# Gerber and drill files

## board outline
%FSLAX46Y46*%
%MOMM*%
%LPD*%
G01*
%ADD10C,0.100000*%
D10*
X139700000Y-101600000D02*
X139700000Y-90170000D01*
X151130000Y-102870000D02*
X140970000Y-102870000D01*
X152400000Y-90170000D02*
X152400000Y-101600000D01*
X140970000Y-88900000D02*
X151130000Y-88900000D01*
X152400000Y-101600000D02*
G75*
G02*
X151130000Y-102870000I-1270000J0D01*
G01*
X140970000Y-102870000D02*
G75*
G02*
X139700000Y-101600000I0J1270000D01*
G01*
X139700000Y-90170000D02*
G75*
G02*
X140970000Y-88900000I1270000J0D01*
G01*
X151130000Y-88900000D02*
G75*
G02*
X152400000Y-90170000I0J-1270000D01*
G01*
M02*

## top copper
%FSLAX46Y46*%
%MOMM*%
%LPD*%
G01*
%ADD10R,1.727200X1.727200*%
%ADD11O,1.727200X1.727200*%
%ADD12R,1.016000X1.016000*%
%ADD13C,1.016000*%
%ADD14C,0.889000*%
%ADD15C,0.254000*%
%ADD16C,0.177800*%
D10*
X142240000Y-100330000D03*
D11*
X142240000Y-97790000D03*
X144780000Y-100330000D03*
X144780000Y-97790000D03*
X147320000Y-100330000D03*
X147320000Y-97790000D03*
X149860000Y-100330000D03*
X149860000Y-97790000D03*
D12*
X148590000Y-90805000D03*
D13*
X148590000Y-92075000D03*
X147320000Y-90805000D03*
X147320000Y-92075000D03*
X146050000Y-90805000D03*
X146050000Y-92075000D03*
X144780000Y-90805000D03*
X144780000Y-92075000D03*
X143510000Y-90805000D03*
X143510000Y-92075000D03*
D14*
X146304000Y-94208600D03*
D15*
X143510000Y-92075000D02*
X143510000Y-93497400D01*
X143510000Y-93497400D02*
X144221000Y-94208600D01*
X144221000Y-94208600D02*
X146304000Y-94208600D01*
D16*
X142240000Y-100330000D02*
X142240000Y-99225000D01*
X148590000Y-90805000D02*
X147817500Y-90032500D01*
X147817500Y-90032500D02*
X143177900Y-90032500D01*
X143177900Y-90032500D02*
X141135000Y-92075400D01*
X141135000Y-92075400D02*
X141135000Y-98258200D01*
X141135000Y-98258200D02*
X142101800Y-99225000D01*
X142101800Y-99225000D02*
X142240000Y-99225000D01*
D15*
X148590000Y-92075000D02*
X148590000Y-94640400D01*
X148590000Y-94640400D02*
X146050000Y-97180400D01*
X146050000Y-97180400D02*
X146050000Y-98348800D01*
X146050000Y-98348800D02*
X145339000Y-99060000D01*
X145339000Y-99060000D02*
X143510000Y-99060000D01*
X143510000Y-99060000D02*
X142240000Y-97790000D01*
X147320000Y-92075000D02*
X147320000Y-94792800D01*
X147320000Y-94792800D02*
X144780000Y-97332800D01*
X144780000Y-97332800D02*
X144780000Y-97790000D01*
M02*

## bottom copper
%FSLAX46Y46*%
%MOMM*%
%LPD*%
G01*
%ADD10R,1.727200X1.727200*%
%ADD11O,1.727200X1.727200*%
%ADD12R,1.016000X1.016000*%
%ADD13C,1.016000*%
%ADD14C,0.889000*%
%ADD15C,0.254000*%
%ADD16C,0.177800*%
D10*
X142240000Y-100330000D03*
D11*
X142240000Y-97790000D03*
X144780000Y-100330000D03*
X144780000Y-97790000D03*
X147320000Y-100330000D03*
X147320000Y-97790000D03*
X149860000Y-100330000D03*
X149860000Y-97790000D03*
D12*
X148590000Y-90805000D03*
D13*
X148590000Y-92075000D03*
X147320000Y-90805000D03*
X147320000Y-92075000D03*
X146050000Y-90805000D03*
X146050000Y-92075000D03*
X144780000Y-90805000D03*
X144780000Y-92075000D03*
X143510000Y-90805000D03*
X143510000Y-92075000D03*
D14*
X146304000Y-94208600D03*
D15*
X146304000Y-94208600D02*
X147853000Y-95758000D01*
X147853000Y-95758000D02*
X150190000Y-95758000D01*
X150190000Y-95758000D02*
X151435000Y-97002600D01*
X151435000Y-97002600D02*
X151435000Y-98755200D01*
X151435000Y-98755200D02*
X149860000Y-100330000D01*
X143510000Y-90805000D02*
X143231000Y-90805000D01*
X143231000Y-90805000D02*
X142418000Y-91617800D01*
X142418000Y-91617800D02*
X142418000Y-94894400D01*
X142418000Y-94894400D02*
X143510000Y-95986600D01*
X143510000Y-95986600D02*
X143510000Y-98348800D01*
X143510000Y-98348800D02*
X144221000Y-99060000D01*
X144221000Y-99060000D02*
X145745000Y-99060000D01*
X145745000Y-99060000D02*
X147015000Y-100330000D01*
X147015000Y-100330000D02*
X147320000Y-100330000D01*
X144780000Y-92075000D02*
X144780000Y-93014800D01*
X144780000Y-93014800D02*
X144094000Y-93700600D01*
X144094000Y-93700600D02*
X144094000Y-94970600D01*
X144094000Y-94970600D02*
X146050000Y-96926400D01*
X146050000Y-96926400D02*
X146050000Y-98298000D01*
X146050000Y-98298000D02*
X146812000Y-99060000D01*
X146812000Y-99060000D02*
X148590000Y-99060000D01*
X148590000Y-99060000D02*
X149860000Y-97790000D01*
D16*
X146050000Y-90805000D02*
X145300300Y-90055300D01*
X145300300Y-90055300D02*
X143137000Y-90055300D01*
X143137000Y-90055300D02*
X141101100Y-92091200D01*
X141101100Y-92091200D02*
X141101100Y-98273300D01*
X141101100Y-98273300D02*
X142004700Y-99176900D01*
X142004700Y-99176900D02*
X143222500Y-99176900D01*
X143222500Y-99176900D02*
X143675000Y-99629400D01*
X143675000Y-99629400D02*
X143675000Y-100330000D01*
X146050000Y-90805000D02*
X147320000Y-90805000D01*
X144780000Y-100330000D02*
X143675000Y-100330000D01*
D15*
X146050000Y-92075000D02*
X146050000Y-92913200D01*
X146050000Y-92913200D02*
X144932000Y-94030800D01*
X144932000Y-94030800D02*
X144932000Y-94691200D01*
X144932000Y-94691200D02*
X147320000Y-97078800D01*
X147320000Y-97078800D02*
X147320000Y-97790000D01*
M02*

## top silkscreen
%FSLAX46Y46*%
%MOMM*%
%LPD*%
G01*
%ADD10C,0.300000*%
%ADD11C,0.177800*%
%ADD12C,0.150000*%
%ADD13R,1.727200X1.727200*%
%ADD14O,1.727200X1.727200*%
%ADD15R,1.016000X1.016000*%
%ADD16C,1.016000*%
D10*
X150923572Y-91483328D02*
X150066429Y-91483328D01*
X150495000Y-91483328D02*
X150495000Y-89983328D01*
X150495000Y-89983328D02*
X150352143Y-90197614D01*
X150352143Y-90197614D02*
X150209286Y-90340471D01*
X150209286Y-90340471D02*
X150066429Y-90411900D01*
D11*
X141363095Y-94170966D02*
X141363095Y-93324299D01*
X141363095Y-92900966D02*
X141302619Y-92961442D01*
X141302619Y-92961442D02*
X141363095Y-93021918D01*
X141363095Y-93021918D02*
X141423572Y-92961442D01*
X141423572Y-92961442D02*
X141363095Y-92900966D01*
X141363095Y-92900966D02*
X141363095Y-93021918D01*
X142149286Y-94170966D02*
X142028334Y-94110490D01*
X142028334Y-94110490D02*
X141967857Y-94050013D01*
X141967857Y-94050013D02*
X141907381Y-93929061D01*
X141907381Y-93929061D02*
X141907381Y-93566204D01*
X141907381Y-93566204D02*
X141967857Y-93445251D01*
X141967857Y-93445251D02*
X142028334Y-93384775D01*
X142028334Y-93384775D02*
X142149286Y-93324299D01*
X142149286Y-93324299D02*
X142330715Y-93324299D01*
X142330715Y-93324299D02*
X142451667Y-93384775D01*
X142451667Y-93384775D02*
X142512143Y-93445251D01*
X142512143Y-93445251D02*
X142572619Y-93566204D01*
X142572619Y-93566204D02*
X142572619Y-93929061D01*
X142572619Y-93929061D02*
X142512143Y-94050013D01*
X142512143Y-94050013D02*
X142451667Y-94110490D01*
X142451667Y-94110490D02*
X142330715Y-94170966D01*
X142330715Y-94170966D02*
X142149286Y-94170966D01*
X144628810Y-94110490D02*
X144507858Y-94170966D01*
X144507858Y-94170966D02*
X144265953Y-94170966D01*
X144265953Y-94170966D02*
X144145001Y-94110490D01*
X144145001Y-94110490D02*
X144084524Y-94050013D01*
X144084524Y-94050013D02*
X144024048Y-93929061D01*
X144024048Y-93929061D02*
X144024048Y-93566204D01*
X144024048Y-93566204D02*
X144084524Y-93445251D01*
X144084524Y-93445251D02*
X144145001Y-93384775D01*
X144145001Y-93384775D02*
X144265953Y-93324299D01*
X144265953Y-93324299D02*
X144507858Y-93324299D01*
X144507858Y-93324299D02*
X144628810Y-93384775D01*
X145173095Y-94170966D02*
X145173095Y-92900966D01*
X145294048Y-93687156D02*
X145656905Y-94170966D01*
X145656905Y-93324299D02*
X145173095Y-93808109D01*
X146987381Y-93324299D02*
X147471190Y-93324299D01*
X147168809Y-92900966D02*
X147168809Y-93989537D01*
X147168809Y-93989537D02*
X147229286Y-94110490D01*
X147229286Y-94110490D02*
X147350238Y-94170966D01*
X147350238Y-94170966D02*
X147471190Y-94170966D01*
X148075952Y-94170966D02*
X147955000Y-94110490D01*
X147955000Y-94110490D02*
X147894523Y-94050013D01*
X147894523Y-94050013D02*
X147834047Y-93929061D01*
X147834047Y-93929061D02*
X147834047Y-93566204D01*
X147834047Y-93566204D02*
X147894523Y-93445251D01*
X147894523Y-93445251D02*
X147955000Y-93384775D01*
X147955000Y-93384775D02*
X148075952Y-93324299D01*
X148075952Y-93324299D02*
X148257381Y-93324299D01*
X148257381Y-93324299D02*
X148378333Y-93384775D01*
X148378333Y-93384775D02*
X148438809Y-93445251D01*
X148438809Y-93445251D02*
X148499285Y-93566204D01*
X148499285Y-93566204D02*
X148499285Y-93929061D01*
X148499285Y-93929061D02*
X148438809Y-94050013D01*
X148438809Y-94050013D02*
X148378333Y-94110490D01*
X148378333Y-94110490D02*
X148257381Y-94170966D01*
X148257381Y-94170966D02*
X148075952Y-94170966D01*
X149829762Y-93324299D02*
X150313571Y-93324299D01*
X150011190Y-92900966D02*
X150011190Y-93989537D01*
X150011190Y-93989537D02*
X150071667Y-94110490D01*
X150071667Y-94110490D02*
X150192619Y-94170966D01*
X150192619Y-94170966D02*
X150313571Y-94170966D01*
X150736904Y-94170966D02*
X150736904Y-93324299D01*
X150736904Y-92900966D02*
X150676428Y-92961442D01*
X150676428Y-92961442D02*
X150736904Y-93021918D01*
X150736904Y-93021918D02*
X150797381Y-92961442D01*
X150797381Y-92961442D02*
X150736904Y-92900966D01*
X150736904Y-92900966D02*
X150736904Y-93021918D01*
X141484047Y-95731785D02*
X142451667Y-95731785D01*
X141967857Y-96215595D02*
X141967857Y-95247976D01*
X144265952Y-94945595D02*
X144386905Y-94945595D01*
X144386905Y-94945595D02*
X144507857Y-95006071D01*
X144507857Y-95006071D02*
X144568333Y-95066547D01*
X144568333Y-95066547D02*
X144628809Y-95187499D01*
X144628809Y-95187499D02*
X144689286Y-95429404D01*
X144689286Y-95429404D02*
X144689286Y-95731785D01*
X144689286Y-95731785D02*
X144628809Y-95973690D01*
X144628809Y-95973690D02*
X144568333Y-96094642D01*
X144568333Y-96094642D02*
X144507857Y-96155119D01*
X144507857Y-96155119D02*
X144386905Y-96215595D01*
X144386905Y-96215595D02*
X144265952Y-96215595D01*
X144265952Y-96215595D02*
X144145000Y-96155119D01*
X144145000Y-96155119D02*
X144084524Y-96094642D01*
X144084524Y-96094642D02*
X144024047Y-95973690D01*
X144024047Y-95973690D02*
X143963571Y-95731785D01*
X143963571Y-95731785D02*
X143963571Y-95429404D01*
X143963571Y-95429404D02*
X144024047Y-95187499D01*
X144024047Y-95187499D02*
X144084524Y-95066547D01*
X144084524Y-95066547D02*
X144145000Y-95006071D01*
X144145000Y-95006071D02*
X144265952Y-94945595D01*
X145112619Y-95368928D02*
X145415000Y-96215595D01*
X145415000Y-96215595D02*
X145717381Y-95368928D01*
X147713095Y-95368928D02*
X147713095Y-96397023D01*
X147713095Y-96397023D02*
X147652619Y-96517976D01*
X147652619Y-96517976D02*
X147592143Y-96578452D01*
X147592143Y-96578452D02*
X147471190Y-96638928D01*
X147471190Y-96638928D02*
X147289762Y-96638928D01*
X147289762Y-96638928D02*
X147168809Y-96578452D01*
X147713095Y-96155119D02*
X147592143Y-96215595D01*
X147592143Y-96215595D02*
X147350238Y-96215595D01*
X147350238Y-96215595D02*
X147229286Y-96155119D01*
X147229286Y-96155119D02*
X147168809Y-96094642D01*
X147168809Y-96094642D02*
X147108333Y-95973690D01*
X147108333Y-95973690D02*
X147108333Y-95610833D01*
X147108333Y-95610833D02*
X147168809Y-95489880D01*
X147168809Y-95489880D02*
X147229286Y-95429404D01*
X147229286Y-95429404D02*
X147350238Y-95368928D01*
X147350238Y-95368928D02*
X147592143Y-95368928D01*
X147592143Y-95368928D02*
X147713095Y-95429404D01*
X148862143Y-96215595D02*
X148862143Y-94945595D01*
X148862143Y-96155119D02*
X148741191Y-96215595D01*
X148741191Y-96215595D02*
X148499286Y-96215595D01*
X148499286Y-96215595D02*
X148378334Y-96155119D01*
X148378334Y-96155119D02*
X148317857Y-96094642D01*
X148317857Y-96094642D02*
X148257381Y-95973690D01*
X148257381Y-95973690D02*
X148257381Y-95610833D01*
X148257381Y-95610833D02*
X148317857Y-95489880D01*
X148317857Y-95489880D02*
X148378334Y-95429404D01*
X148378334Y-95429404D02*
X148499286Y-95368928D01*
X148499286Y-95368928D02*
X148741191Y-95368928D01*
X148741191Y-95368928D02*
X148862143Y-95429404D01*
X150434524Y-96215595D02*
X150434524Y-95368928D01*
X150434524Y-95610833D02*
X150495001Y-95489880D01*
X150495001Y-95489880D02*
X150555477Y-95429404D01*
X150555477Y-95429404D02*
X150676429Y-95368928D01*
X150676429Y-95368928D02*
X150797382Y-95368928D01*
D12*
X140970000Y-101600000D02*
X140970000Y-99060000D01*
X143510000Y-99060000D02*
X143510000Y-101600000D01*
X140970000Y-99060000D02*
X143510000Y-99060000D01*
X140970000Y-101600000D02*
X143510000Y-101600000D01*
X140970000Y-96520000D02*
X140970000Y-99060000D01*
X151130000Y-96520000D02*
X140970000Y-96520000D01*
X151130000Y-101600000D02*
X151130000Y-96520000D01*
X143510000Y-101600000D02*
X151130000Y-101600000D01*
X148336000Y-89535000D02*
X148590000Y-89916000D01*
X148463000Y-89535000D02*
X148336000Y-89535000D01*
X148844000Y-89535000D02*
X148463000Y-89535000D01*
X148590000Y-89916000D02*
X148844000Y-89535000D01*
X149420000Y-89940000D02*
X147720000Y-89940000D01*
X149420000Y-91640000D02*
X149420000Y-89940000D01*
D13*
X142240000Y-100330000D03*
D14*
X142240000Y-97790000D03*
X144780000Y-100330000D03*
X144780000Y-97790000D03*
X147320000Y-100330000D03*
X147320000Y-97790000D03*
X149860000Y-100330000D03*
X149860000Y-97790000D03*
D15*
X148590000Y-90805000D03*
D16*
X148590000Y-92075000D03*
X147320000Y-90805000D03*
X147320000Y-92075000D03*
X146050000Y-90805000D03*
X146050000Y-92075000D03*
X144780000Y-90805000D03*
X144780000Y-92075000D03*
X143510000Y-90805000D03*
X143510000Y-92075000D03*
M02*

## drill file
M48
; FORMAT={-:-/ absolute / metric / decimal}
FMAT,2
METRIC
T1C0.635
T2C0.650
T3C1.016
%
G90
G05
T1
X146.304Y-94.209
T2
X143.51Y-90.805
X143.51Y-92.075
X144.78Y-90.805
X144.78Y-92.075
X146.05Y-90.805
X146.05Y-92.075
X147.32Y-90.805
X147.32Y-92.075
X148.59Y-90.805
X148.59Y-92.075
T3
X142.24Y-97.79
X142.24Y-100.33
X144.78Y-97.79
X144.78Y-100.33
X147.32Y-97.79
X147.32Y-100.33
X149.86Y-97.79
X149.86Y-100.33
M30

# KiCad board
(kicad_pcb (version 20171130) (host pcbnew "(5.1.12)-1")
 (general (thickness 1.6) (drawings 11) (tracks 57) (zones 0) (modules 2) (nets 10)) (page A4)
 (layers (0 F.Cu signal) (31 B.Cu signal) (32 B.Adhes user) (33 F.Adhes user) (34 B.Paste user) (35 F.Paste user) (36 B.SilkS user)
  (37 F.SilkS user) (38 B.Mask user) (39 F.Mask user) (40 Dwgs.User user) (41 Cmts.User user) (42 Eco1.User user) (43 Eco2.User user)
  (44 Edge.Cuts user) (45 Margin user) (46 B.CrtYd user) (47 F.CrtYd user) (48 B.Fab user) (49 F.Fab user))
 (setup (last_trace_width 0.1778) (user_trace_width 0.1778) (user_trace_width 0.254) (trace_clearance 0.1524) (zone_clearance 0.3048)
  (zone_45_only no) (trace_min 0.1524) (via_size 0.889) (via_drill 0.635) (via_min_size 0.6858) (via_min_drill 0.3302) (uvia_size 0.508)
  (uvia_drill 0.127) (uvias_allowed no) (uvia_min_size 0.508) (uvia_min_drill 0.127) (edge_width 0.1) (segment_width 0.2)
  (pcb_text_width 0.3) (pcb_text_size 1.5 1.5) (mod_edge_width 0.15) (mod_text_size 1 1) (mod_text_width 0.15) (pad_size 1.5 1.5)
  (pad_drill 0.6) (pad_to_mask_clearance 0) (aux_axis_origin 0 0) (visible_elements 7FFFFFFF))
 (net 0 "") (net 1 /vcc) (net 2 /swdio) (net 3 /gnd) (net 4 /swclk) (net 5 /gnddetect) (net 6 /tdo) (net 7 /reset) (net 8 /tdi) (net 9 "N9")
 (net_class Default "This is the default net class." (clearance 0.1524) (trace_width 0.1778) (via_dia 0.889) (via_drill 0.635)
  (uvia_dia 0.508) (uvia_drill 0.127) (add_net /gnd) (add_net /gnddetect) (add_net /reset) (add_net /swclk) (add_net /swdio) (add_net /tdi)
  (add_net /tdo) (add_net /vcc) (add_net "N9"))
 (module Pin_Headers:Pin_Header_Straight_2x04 (layer F.Cu) (at 146.05 99.06)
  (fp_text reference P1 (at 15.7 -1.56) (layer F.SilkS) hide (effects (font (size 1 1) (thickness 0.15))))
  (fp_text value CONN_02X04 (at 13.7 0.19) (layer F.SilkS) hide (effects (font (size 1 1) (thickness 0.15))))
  (fp_line (start -5.08 2.54) (end -5.08 0) (layer F.SilkS) (width 0.15))
  (fp_line (start -2.54 0) (end -2.54 2.54) (layer F.SilkS) (width 0.15))
  (fp_line (start -5.08 0) (end -2.54 0) (layer F.SilkS) (width 0.15))
  (fp_line (start -5.08 2.54) (end -2.54 2.54) (layer F.SilkS) (width 0.15))
  (fp_line (start -5.08 -2.54) (end -5.08 0) (layer F.SilkS) (width 0.15))
  (fp_line (start 5.08 -2.54) (end -5.08 -2.54) (layer F.SilkS) (width 0.15))
  (fp_line (start 5.08 2.54) (end 5.08 -2.54) (layer F.SilkS) (width 0.15))
  (fp_line (start -2.54 2.54) (end 5.08 2.54) (layer F.SilkS) (width 0.15))
  (pad 1 thru_hole rect (at -3.81 1.27) (size 1.7272 1.7272) (drill 1.016) (layers *.Cu *.Mask F.SilkS) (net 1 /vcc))
  (pad 2 thru_hole oval (at -3.81 -1.27) (size 1.7272 1.7272) (drill 1.016) (layers *.Cu *.Mask F.SilkS) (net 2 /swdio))
  (pad 3 thru_hole oval (at -1.27 1.27) (size 1.7272 1.7272) (drill 1.016) (layers *.Cu *.Mask F.SilkS) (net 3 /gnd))
  (pad 4 thru_hole oval (at -1.27 -1.27) (size 1.7272 1.7272) (drill 1.016) (layers *.Cu *.Mask F.SilkS) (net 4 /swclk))
  (pad 5 thru_hole oval (at 1.27 1.27) (size 1.7272 1.7272) (drill 1.016) (layers *.Cu *.Mask F.SilkS) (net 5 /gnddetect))
  (pad 6 thru_hole oval (at 1.27 -1.27) (size 1.7272 1.7272) (drill 1.016) (layers *.Cu *.Mask F.SilkS) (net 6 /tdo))
  (pad 7 thru_hole oval (at 3.81 1.27) (size 1.7272 1.7272) (drill 1.016) (layers *.Cu *.Mask F.SilkS) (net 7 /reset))
  (pad 8 thru_hole oval (at 3.81 -1.27) (size 1.7272 1.7272) (drill 1.016) (layers *.Cu *.Mask F.SilkS) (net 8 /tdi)))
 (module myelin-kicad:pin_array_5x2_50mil (layer F.Cu) (at 147.32 91.44 180)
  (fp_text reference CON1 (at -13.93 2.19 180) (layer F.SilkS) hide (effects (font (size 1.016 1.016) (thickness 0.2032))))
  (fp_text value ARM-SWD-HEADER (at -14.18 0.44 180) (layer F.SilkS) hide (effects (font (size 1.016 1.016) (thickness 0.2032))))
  (fp_line (start -1.016 1.905) (end -1.27 1.524) (layer F.SilkS) (width 0.15))
  (fp_line (start -1.143 1.905) (end -1.016 1.905) (layer F.SilkS) (width 0.15))
  (fp_line (start -1.524 1.905) (end -1.143 1.905) (layer F.SilkS) (width 0.15))
  (fp_line (start -1.27 1.524) (end -1.524 1.905) (layer F.SilkS) (width 0.15))
  (fp_line (start -2.1 1.5) (end -0.4 1.5) (layer F.SilkS) (width 0.15))
  (fp_line (start -2.1 -0.2) (end -2.1 1.5) (layer F.SilkS) (width 0.15))
  (pad 1 thru_hole rect (at -1.27 0.635 180) (size 1.016 1.016) (drill 0.65) (layers *.Cu *.Mask F.SilkS) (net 1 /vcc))
  (pad 2 thru_hole circle (at -1.27 -0.635 180) (size 1.016 1.016) (drill 0.65) (layers *.Cu *.Mask F.SilkS) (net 2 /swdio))
  (pad 3 thru_hole circle (at 0 0.635 180) (size 1.016 1.016) (drill 0.65) (layers *.Cu *.Mask F.SilkS) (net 3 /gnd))
  (pad 4 thru_hole circle (at 0 -0.635 180) (size 1.016 1.016) (drill 0.65) (layers *.Cu *.Mask F.SilkS) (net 4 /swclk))
  (pad 5 thru_hole circle (at 1.27 0.635 180) (size 1.016 1.016) (drill 0.65) (layers *.Cu *.Mask F.SilkS) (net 3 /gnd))
  (pad 6 thru_hole circle (at 1.27 -0.635 180) (size 1.016 1.016) (drill 0.65) (layers *.Cu *.Mask F.SilkS) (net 6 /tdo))
  (pad 7 thru_hole circle (at 2.54 0.635 180) (size 1.016 1.016) (drill 0.65) (layers *.Cu *.Mask F.SilkS) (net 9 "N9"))
  (pad 8 thru_hole circle (at 2.54 -0.635 180) (size 1.016 1.016) (drill 0.65) (layers *.Cu *.Mask F.SilkS) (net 8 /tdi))
  (pad 9 thru_hole circle (at 3.81 0.635 180) (size 1.016 1.016) (drill 0.65) (layers *.Cu *.Mask F.SilkS) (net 5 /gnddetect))
  (pad 10 thru_hole circle (at 3.81 -0.635 180) (size 1.016 1.016) (drill 0.65) (layers *.Cu *.Mask F.SilkS) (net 7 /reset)))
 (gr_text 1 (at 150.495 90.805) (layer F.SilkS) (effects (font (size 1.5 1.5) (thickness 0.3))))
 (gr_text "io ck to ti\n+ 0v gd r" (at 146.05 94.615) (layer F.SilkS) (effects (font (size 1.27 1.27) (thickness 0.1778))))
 (gr_line (start 139.7 101.6) (end 139.7 90.17) (angle 90) (layer Edge.Cuts) (width 0.1))
 (gr_line (start 151.13 102.87) (end 140.97 102.87) (angle 90) (layer Edge.Cuts) (width 0.1))
 (gr_line (start 152.4 90.17) (end 152.4 101.6) (angle 90) (layer Edge.Cuts) (width 0.1))
 (gr_line (start 140.97 88.9) (end 151.13 88.9) (angle 90) (layer Edge.Cuts) (width 0.1))
 (gr_arc (start 151.13 101.6) (end 152.4 101.6) (angle 90) (layer Edge.Cuts) (width 0.1))
 (gr_arc (start 140.97 101.6) (end 140.97 102.87) (angle 90) (layer Edge.Cuts) (width 0.1))
 (gr_arc (start 140.97 90.17) (end 139.7 90.17) (angle 90) (layer Edge.Cuts) (width 0.1))
 (gr_arc (start 151.13 90.17) (end 151.13 88.9) (angle 90) (layer Edge.Cuts) (width 0.1))
 (segment (start 143.51 92.075) (end 143.51 93.4974) (width 0.254) (layer F.Cu) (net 7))
 (segment (start 143.51 93.4974) (end 144.221 94.2086) (width 0.254) (layer F.Cu) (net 7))
 (segment (start 144.221 94.2086) (end 146.304 94.2086) (width 0.254) (layer F.Cu) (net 7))
 (segment (start 146.304 94.2086) (end 147.853 95.758) (width 0.254) (layer B.Cu) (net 7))
 (segment (start 147.853 95.758) (end 150.19 95.758) (width 0.254) (layer B.Cu) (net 7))
 (segment (start 150.19 95.758) (end 151.435 97.0026) (width 0.254) (layer B.Cu) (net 7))
 (segment (start 151.435 97.0026) (end 151.435 98.7552) (width 0.254) (layer B.Cu) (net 7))
 (segment (start 151.435 98.7552) (end 149.86 100.33) (width 0.254) (layer B.Cu) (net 7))
 (via (at 146.304 94.2086) (size 0.889) (layers F.Cu B.Cu) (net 7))
 (segment (start 143.51 90.805) (end 143.231 90.805) (width 0.254) (layer B.Cu) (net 5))
 (segment (start 143.231 90.805) (end 142.418 91.6178) (width 0.254) (layer B.Cu) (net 5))
 (segment (start 142.418 91.6178) (end 142.418 94.8944) (width 0.254) (layer B.Cu) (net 5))
 (segment (start 142.418 94.8944) (end 143.51 95.9866) (width 0.254) (layer B.Cu) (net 5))
 (segment (start 143.51 95.9866) (end 143.51 98.3488) (width 0.254) (layer B.Cu) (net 5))
 (segment (start 143.51 98.3488) (end 144.221 99.06) (width 0.254) (layer B.Cu) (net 5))
 (segment (start 144.221 99.06) (end 145.745 99.06) (width 0.254) (layer B.Cu) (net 5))
 (segment (start 145.745 99.06) (end 147.015 100.33) (width 0.254) (layer B.Cu) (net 5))
 (segment (start 147.015 100.33) (end 147.32 100.33) (width 0.254) (layer B.Cu) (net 5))
 (segment (start 144.78 92.075) (end 144.78 93.0148) (width 0.254) (layer B.Cu) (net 8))
 (segment (start 144.78 93.0148) (end 144.094 93.7006) (width 0.254) (layer B.Cu) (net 8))
 (segment (start 144.094 93.7006) (end 144.094 94.9706) (width 0.254) (layer B.Cu) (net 8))
 (segment (start 144.094 94.9706) (end 146.05 96.9264) (width 0.254) (layer B.Cu) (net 8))
 (segment (start 146.05 96.9264) (end 146.05 98.298) (width 0.254) (layer B.Cu) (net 8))
 (segment (start 146.05 98.298) (end 146.812 99.06) (width 0.254) (layer B.Cu) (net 8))
 (segment (start 146.812 99.06) (end 148.59 99.06) (width 0.254) (layer B.Cu) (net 8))
 (segment (start 148.59 99.06) (end 149.86 97.79) (width 0.254) (layer B.Cu) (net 8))
 (segment (start 142.24 100.33) (end 142.24 99.225) (width 0.1778) (layer F.Cu) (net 1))
 (segment (start 148.59 90.805) (end 147.8175 90.0325) (width 0.1778) (layer F.Cu) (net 1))
 (segment (start 147.8175 90.0325) (end 143.1779 90.0325) (width 0.1778) (layer F.Cu) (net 1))
 (segment (start 143.1779 90.0325) (end 141.135 92.0754) (width 0.1778) (layer F.Cu) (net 1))
 (segment (start 141.135 92.0754) (end 141.135 98.2582) (width 0.1778) (layer F.Cu) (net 1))
 (segment (start 141.135 98.2582) (end 142.1018 99.225) (width 0.1778) (layer F.Cu) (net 1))
 (segment (start 142.1018 99.225) (end 142.24 99.225) (width 0.1778) (layer F.Cu) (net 1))
 (segment (start 148.59 92.075) (end 148.59 94.6404) (width 0.254) (layer F.Cu) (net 2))
 (segment (start 148.59 94.6404) (end 146.05 97.1804) (width 0.254) (layer F.Cu) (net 2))
 (segment (start 146.05 97.1804) (end 146.05 98.3488) (width 0.254) (layer F.Cu) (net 2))
 (segment (start 146.05 98.3488) (end 145.339 99.06) (width 0.254) (layer F.Cu) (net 2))
 (segment (start 145.339 99.06) (end 143.51 99.06) (width 0.254) (layer F.Cu) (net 2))
 (segment (start 143.51 99.06) (end 142.24 97.79) (width 0.254) (layer F.Cu) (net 2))
 (segment (start 146.05 90.805) (end 145.3003 90.0553) (width 0.1778) (layer B.Cu) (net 3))
 (segment (start 145.3003 90.0553) (end 143.137 90.0553) (width 0.1778) (layer B.Cu) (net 3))
 (segment (start 143.137 90.0553) (end 141.1011 92.0912) (width 0.1778) (layer B.Cu) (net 3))
 (segment (start 141.1011 92.0912) (end 141.1011 98.2733) (width 0.1778) (layer B.Cu) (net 3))
 (segment (start 141.1011 98.2733) (end 142.0047 99.1769) (width 0.1778) (layer B.Cu) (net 3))
 (segment (start 142.0047 99.1769) (end 143.2225 99.1769) (width 0.1778) (layer B.Cu) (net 3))
 (segment (start 143.2225 99.1769) (end 143.675 99.6294) (width 0.1778) (layer B.Cu) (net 3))
 (segment (start 143.675 99.6294) (end 143.675 100.33) (width 0.1778) (layer B.Cu) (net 3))
 (segment (start 146.05 90.805) (end 147.32 90.805) (width 0.1778) (layer B.Cu) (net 3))
 (segment (start 144.78 100.33) (end 143.675 100.33) (width 0.1778) (layer B.Cu) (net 3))
 (segment (start 147.32 92.075) (end 147.32 94.7928) (width 0.254) (layer F.Cu) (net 4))
 (segment (start 147.32 94.7928) (end 144.78 97.3328) (width 0.254) (layer F.Cu) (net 4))
 (segment (start 144.78 97.3328) (end 144.78 97.79) (width 0.254) (layer F.Cu) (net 4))
 (segment (start 146.05 92.075) (end 146.05 92.9132) (width 0.254) (layer B.Cu) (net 6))
 (segment (start 146.05 92.9132) (end 144.932 94.0308) (width 0.254) (layer B.Cu) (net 6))
 (segment (start 144.932 94.0308) (end 144.932 94.6912) (width 0.254) (layer B.Cu) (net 6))
 (segment (start 144.932 94.6912) (end 147.32 97.0788) (width 0.254) (layer B.Cu) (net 6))
 (segment (start 147.32 97.0788) (end 147.32 97.79) (width 0.254) (layer B.Cu) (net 6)))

